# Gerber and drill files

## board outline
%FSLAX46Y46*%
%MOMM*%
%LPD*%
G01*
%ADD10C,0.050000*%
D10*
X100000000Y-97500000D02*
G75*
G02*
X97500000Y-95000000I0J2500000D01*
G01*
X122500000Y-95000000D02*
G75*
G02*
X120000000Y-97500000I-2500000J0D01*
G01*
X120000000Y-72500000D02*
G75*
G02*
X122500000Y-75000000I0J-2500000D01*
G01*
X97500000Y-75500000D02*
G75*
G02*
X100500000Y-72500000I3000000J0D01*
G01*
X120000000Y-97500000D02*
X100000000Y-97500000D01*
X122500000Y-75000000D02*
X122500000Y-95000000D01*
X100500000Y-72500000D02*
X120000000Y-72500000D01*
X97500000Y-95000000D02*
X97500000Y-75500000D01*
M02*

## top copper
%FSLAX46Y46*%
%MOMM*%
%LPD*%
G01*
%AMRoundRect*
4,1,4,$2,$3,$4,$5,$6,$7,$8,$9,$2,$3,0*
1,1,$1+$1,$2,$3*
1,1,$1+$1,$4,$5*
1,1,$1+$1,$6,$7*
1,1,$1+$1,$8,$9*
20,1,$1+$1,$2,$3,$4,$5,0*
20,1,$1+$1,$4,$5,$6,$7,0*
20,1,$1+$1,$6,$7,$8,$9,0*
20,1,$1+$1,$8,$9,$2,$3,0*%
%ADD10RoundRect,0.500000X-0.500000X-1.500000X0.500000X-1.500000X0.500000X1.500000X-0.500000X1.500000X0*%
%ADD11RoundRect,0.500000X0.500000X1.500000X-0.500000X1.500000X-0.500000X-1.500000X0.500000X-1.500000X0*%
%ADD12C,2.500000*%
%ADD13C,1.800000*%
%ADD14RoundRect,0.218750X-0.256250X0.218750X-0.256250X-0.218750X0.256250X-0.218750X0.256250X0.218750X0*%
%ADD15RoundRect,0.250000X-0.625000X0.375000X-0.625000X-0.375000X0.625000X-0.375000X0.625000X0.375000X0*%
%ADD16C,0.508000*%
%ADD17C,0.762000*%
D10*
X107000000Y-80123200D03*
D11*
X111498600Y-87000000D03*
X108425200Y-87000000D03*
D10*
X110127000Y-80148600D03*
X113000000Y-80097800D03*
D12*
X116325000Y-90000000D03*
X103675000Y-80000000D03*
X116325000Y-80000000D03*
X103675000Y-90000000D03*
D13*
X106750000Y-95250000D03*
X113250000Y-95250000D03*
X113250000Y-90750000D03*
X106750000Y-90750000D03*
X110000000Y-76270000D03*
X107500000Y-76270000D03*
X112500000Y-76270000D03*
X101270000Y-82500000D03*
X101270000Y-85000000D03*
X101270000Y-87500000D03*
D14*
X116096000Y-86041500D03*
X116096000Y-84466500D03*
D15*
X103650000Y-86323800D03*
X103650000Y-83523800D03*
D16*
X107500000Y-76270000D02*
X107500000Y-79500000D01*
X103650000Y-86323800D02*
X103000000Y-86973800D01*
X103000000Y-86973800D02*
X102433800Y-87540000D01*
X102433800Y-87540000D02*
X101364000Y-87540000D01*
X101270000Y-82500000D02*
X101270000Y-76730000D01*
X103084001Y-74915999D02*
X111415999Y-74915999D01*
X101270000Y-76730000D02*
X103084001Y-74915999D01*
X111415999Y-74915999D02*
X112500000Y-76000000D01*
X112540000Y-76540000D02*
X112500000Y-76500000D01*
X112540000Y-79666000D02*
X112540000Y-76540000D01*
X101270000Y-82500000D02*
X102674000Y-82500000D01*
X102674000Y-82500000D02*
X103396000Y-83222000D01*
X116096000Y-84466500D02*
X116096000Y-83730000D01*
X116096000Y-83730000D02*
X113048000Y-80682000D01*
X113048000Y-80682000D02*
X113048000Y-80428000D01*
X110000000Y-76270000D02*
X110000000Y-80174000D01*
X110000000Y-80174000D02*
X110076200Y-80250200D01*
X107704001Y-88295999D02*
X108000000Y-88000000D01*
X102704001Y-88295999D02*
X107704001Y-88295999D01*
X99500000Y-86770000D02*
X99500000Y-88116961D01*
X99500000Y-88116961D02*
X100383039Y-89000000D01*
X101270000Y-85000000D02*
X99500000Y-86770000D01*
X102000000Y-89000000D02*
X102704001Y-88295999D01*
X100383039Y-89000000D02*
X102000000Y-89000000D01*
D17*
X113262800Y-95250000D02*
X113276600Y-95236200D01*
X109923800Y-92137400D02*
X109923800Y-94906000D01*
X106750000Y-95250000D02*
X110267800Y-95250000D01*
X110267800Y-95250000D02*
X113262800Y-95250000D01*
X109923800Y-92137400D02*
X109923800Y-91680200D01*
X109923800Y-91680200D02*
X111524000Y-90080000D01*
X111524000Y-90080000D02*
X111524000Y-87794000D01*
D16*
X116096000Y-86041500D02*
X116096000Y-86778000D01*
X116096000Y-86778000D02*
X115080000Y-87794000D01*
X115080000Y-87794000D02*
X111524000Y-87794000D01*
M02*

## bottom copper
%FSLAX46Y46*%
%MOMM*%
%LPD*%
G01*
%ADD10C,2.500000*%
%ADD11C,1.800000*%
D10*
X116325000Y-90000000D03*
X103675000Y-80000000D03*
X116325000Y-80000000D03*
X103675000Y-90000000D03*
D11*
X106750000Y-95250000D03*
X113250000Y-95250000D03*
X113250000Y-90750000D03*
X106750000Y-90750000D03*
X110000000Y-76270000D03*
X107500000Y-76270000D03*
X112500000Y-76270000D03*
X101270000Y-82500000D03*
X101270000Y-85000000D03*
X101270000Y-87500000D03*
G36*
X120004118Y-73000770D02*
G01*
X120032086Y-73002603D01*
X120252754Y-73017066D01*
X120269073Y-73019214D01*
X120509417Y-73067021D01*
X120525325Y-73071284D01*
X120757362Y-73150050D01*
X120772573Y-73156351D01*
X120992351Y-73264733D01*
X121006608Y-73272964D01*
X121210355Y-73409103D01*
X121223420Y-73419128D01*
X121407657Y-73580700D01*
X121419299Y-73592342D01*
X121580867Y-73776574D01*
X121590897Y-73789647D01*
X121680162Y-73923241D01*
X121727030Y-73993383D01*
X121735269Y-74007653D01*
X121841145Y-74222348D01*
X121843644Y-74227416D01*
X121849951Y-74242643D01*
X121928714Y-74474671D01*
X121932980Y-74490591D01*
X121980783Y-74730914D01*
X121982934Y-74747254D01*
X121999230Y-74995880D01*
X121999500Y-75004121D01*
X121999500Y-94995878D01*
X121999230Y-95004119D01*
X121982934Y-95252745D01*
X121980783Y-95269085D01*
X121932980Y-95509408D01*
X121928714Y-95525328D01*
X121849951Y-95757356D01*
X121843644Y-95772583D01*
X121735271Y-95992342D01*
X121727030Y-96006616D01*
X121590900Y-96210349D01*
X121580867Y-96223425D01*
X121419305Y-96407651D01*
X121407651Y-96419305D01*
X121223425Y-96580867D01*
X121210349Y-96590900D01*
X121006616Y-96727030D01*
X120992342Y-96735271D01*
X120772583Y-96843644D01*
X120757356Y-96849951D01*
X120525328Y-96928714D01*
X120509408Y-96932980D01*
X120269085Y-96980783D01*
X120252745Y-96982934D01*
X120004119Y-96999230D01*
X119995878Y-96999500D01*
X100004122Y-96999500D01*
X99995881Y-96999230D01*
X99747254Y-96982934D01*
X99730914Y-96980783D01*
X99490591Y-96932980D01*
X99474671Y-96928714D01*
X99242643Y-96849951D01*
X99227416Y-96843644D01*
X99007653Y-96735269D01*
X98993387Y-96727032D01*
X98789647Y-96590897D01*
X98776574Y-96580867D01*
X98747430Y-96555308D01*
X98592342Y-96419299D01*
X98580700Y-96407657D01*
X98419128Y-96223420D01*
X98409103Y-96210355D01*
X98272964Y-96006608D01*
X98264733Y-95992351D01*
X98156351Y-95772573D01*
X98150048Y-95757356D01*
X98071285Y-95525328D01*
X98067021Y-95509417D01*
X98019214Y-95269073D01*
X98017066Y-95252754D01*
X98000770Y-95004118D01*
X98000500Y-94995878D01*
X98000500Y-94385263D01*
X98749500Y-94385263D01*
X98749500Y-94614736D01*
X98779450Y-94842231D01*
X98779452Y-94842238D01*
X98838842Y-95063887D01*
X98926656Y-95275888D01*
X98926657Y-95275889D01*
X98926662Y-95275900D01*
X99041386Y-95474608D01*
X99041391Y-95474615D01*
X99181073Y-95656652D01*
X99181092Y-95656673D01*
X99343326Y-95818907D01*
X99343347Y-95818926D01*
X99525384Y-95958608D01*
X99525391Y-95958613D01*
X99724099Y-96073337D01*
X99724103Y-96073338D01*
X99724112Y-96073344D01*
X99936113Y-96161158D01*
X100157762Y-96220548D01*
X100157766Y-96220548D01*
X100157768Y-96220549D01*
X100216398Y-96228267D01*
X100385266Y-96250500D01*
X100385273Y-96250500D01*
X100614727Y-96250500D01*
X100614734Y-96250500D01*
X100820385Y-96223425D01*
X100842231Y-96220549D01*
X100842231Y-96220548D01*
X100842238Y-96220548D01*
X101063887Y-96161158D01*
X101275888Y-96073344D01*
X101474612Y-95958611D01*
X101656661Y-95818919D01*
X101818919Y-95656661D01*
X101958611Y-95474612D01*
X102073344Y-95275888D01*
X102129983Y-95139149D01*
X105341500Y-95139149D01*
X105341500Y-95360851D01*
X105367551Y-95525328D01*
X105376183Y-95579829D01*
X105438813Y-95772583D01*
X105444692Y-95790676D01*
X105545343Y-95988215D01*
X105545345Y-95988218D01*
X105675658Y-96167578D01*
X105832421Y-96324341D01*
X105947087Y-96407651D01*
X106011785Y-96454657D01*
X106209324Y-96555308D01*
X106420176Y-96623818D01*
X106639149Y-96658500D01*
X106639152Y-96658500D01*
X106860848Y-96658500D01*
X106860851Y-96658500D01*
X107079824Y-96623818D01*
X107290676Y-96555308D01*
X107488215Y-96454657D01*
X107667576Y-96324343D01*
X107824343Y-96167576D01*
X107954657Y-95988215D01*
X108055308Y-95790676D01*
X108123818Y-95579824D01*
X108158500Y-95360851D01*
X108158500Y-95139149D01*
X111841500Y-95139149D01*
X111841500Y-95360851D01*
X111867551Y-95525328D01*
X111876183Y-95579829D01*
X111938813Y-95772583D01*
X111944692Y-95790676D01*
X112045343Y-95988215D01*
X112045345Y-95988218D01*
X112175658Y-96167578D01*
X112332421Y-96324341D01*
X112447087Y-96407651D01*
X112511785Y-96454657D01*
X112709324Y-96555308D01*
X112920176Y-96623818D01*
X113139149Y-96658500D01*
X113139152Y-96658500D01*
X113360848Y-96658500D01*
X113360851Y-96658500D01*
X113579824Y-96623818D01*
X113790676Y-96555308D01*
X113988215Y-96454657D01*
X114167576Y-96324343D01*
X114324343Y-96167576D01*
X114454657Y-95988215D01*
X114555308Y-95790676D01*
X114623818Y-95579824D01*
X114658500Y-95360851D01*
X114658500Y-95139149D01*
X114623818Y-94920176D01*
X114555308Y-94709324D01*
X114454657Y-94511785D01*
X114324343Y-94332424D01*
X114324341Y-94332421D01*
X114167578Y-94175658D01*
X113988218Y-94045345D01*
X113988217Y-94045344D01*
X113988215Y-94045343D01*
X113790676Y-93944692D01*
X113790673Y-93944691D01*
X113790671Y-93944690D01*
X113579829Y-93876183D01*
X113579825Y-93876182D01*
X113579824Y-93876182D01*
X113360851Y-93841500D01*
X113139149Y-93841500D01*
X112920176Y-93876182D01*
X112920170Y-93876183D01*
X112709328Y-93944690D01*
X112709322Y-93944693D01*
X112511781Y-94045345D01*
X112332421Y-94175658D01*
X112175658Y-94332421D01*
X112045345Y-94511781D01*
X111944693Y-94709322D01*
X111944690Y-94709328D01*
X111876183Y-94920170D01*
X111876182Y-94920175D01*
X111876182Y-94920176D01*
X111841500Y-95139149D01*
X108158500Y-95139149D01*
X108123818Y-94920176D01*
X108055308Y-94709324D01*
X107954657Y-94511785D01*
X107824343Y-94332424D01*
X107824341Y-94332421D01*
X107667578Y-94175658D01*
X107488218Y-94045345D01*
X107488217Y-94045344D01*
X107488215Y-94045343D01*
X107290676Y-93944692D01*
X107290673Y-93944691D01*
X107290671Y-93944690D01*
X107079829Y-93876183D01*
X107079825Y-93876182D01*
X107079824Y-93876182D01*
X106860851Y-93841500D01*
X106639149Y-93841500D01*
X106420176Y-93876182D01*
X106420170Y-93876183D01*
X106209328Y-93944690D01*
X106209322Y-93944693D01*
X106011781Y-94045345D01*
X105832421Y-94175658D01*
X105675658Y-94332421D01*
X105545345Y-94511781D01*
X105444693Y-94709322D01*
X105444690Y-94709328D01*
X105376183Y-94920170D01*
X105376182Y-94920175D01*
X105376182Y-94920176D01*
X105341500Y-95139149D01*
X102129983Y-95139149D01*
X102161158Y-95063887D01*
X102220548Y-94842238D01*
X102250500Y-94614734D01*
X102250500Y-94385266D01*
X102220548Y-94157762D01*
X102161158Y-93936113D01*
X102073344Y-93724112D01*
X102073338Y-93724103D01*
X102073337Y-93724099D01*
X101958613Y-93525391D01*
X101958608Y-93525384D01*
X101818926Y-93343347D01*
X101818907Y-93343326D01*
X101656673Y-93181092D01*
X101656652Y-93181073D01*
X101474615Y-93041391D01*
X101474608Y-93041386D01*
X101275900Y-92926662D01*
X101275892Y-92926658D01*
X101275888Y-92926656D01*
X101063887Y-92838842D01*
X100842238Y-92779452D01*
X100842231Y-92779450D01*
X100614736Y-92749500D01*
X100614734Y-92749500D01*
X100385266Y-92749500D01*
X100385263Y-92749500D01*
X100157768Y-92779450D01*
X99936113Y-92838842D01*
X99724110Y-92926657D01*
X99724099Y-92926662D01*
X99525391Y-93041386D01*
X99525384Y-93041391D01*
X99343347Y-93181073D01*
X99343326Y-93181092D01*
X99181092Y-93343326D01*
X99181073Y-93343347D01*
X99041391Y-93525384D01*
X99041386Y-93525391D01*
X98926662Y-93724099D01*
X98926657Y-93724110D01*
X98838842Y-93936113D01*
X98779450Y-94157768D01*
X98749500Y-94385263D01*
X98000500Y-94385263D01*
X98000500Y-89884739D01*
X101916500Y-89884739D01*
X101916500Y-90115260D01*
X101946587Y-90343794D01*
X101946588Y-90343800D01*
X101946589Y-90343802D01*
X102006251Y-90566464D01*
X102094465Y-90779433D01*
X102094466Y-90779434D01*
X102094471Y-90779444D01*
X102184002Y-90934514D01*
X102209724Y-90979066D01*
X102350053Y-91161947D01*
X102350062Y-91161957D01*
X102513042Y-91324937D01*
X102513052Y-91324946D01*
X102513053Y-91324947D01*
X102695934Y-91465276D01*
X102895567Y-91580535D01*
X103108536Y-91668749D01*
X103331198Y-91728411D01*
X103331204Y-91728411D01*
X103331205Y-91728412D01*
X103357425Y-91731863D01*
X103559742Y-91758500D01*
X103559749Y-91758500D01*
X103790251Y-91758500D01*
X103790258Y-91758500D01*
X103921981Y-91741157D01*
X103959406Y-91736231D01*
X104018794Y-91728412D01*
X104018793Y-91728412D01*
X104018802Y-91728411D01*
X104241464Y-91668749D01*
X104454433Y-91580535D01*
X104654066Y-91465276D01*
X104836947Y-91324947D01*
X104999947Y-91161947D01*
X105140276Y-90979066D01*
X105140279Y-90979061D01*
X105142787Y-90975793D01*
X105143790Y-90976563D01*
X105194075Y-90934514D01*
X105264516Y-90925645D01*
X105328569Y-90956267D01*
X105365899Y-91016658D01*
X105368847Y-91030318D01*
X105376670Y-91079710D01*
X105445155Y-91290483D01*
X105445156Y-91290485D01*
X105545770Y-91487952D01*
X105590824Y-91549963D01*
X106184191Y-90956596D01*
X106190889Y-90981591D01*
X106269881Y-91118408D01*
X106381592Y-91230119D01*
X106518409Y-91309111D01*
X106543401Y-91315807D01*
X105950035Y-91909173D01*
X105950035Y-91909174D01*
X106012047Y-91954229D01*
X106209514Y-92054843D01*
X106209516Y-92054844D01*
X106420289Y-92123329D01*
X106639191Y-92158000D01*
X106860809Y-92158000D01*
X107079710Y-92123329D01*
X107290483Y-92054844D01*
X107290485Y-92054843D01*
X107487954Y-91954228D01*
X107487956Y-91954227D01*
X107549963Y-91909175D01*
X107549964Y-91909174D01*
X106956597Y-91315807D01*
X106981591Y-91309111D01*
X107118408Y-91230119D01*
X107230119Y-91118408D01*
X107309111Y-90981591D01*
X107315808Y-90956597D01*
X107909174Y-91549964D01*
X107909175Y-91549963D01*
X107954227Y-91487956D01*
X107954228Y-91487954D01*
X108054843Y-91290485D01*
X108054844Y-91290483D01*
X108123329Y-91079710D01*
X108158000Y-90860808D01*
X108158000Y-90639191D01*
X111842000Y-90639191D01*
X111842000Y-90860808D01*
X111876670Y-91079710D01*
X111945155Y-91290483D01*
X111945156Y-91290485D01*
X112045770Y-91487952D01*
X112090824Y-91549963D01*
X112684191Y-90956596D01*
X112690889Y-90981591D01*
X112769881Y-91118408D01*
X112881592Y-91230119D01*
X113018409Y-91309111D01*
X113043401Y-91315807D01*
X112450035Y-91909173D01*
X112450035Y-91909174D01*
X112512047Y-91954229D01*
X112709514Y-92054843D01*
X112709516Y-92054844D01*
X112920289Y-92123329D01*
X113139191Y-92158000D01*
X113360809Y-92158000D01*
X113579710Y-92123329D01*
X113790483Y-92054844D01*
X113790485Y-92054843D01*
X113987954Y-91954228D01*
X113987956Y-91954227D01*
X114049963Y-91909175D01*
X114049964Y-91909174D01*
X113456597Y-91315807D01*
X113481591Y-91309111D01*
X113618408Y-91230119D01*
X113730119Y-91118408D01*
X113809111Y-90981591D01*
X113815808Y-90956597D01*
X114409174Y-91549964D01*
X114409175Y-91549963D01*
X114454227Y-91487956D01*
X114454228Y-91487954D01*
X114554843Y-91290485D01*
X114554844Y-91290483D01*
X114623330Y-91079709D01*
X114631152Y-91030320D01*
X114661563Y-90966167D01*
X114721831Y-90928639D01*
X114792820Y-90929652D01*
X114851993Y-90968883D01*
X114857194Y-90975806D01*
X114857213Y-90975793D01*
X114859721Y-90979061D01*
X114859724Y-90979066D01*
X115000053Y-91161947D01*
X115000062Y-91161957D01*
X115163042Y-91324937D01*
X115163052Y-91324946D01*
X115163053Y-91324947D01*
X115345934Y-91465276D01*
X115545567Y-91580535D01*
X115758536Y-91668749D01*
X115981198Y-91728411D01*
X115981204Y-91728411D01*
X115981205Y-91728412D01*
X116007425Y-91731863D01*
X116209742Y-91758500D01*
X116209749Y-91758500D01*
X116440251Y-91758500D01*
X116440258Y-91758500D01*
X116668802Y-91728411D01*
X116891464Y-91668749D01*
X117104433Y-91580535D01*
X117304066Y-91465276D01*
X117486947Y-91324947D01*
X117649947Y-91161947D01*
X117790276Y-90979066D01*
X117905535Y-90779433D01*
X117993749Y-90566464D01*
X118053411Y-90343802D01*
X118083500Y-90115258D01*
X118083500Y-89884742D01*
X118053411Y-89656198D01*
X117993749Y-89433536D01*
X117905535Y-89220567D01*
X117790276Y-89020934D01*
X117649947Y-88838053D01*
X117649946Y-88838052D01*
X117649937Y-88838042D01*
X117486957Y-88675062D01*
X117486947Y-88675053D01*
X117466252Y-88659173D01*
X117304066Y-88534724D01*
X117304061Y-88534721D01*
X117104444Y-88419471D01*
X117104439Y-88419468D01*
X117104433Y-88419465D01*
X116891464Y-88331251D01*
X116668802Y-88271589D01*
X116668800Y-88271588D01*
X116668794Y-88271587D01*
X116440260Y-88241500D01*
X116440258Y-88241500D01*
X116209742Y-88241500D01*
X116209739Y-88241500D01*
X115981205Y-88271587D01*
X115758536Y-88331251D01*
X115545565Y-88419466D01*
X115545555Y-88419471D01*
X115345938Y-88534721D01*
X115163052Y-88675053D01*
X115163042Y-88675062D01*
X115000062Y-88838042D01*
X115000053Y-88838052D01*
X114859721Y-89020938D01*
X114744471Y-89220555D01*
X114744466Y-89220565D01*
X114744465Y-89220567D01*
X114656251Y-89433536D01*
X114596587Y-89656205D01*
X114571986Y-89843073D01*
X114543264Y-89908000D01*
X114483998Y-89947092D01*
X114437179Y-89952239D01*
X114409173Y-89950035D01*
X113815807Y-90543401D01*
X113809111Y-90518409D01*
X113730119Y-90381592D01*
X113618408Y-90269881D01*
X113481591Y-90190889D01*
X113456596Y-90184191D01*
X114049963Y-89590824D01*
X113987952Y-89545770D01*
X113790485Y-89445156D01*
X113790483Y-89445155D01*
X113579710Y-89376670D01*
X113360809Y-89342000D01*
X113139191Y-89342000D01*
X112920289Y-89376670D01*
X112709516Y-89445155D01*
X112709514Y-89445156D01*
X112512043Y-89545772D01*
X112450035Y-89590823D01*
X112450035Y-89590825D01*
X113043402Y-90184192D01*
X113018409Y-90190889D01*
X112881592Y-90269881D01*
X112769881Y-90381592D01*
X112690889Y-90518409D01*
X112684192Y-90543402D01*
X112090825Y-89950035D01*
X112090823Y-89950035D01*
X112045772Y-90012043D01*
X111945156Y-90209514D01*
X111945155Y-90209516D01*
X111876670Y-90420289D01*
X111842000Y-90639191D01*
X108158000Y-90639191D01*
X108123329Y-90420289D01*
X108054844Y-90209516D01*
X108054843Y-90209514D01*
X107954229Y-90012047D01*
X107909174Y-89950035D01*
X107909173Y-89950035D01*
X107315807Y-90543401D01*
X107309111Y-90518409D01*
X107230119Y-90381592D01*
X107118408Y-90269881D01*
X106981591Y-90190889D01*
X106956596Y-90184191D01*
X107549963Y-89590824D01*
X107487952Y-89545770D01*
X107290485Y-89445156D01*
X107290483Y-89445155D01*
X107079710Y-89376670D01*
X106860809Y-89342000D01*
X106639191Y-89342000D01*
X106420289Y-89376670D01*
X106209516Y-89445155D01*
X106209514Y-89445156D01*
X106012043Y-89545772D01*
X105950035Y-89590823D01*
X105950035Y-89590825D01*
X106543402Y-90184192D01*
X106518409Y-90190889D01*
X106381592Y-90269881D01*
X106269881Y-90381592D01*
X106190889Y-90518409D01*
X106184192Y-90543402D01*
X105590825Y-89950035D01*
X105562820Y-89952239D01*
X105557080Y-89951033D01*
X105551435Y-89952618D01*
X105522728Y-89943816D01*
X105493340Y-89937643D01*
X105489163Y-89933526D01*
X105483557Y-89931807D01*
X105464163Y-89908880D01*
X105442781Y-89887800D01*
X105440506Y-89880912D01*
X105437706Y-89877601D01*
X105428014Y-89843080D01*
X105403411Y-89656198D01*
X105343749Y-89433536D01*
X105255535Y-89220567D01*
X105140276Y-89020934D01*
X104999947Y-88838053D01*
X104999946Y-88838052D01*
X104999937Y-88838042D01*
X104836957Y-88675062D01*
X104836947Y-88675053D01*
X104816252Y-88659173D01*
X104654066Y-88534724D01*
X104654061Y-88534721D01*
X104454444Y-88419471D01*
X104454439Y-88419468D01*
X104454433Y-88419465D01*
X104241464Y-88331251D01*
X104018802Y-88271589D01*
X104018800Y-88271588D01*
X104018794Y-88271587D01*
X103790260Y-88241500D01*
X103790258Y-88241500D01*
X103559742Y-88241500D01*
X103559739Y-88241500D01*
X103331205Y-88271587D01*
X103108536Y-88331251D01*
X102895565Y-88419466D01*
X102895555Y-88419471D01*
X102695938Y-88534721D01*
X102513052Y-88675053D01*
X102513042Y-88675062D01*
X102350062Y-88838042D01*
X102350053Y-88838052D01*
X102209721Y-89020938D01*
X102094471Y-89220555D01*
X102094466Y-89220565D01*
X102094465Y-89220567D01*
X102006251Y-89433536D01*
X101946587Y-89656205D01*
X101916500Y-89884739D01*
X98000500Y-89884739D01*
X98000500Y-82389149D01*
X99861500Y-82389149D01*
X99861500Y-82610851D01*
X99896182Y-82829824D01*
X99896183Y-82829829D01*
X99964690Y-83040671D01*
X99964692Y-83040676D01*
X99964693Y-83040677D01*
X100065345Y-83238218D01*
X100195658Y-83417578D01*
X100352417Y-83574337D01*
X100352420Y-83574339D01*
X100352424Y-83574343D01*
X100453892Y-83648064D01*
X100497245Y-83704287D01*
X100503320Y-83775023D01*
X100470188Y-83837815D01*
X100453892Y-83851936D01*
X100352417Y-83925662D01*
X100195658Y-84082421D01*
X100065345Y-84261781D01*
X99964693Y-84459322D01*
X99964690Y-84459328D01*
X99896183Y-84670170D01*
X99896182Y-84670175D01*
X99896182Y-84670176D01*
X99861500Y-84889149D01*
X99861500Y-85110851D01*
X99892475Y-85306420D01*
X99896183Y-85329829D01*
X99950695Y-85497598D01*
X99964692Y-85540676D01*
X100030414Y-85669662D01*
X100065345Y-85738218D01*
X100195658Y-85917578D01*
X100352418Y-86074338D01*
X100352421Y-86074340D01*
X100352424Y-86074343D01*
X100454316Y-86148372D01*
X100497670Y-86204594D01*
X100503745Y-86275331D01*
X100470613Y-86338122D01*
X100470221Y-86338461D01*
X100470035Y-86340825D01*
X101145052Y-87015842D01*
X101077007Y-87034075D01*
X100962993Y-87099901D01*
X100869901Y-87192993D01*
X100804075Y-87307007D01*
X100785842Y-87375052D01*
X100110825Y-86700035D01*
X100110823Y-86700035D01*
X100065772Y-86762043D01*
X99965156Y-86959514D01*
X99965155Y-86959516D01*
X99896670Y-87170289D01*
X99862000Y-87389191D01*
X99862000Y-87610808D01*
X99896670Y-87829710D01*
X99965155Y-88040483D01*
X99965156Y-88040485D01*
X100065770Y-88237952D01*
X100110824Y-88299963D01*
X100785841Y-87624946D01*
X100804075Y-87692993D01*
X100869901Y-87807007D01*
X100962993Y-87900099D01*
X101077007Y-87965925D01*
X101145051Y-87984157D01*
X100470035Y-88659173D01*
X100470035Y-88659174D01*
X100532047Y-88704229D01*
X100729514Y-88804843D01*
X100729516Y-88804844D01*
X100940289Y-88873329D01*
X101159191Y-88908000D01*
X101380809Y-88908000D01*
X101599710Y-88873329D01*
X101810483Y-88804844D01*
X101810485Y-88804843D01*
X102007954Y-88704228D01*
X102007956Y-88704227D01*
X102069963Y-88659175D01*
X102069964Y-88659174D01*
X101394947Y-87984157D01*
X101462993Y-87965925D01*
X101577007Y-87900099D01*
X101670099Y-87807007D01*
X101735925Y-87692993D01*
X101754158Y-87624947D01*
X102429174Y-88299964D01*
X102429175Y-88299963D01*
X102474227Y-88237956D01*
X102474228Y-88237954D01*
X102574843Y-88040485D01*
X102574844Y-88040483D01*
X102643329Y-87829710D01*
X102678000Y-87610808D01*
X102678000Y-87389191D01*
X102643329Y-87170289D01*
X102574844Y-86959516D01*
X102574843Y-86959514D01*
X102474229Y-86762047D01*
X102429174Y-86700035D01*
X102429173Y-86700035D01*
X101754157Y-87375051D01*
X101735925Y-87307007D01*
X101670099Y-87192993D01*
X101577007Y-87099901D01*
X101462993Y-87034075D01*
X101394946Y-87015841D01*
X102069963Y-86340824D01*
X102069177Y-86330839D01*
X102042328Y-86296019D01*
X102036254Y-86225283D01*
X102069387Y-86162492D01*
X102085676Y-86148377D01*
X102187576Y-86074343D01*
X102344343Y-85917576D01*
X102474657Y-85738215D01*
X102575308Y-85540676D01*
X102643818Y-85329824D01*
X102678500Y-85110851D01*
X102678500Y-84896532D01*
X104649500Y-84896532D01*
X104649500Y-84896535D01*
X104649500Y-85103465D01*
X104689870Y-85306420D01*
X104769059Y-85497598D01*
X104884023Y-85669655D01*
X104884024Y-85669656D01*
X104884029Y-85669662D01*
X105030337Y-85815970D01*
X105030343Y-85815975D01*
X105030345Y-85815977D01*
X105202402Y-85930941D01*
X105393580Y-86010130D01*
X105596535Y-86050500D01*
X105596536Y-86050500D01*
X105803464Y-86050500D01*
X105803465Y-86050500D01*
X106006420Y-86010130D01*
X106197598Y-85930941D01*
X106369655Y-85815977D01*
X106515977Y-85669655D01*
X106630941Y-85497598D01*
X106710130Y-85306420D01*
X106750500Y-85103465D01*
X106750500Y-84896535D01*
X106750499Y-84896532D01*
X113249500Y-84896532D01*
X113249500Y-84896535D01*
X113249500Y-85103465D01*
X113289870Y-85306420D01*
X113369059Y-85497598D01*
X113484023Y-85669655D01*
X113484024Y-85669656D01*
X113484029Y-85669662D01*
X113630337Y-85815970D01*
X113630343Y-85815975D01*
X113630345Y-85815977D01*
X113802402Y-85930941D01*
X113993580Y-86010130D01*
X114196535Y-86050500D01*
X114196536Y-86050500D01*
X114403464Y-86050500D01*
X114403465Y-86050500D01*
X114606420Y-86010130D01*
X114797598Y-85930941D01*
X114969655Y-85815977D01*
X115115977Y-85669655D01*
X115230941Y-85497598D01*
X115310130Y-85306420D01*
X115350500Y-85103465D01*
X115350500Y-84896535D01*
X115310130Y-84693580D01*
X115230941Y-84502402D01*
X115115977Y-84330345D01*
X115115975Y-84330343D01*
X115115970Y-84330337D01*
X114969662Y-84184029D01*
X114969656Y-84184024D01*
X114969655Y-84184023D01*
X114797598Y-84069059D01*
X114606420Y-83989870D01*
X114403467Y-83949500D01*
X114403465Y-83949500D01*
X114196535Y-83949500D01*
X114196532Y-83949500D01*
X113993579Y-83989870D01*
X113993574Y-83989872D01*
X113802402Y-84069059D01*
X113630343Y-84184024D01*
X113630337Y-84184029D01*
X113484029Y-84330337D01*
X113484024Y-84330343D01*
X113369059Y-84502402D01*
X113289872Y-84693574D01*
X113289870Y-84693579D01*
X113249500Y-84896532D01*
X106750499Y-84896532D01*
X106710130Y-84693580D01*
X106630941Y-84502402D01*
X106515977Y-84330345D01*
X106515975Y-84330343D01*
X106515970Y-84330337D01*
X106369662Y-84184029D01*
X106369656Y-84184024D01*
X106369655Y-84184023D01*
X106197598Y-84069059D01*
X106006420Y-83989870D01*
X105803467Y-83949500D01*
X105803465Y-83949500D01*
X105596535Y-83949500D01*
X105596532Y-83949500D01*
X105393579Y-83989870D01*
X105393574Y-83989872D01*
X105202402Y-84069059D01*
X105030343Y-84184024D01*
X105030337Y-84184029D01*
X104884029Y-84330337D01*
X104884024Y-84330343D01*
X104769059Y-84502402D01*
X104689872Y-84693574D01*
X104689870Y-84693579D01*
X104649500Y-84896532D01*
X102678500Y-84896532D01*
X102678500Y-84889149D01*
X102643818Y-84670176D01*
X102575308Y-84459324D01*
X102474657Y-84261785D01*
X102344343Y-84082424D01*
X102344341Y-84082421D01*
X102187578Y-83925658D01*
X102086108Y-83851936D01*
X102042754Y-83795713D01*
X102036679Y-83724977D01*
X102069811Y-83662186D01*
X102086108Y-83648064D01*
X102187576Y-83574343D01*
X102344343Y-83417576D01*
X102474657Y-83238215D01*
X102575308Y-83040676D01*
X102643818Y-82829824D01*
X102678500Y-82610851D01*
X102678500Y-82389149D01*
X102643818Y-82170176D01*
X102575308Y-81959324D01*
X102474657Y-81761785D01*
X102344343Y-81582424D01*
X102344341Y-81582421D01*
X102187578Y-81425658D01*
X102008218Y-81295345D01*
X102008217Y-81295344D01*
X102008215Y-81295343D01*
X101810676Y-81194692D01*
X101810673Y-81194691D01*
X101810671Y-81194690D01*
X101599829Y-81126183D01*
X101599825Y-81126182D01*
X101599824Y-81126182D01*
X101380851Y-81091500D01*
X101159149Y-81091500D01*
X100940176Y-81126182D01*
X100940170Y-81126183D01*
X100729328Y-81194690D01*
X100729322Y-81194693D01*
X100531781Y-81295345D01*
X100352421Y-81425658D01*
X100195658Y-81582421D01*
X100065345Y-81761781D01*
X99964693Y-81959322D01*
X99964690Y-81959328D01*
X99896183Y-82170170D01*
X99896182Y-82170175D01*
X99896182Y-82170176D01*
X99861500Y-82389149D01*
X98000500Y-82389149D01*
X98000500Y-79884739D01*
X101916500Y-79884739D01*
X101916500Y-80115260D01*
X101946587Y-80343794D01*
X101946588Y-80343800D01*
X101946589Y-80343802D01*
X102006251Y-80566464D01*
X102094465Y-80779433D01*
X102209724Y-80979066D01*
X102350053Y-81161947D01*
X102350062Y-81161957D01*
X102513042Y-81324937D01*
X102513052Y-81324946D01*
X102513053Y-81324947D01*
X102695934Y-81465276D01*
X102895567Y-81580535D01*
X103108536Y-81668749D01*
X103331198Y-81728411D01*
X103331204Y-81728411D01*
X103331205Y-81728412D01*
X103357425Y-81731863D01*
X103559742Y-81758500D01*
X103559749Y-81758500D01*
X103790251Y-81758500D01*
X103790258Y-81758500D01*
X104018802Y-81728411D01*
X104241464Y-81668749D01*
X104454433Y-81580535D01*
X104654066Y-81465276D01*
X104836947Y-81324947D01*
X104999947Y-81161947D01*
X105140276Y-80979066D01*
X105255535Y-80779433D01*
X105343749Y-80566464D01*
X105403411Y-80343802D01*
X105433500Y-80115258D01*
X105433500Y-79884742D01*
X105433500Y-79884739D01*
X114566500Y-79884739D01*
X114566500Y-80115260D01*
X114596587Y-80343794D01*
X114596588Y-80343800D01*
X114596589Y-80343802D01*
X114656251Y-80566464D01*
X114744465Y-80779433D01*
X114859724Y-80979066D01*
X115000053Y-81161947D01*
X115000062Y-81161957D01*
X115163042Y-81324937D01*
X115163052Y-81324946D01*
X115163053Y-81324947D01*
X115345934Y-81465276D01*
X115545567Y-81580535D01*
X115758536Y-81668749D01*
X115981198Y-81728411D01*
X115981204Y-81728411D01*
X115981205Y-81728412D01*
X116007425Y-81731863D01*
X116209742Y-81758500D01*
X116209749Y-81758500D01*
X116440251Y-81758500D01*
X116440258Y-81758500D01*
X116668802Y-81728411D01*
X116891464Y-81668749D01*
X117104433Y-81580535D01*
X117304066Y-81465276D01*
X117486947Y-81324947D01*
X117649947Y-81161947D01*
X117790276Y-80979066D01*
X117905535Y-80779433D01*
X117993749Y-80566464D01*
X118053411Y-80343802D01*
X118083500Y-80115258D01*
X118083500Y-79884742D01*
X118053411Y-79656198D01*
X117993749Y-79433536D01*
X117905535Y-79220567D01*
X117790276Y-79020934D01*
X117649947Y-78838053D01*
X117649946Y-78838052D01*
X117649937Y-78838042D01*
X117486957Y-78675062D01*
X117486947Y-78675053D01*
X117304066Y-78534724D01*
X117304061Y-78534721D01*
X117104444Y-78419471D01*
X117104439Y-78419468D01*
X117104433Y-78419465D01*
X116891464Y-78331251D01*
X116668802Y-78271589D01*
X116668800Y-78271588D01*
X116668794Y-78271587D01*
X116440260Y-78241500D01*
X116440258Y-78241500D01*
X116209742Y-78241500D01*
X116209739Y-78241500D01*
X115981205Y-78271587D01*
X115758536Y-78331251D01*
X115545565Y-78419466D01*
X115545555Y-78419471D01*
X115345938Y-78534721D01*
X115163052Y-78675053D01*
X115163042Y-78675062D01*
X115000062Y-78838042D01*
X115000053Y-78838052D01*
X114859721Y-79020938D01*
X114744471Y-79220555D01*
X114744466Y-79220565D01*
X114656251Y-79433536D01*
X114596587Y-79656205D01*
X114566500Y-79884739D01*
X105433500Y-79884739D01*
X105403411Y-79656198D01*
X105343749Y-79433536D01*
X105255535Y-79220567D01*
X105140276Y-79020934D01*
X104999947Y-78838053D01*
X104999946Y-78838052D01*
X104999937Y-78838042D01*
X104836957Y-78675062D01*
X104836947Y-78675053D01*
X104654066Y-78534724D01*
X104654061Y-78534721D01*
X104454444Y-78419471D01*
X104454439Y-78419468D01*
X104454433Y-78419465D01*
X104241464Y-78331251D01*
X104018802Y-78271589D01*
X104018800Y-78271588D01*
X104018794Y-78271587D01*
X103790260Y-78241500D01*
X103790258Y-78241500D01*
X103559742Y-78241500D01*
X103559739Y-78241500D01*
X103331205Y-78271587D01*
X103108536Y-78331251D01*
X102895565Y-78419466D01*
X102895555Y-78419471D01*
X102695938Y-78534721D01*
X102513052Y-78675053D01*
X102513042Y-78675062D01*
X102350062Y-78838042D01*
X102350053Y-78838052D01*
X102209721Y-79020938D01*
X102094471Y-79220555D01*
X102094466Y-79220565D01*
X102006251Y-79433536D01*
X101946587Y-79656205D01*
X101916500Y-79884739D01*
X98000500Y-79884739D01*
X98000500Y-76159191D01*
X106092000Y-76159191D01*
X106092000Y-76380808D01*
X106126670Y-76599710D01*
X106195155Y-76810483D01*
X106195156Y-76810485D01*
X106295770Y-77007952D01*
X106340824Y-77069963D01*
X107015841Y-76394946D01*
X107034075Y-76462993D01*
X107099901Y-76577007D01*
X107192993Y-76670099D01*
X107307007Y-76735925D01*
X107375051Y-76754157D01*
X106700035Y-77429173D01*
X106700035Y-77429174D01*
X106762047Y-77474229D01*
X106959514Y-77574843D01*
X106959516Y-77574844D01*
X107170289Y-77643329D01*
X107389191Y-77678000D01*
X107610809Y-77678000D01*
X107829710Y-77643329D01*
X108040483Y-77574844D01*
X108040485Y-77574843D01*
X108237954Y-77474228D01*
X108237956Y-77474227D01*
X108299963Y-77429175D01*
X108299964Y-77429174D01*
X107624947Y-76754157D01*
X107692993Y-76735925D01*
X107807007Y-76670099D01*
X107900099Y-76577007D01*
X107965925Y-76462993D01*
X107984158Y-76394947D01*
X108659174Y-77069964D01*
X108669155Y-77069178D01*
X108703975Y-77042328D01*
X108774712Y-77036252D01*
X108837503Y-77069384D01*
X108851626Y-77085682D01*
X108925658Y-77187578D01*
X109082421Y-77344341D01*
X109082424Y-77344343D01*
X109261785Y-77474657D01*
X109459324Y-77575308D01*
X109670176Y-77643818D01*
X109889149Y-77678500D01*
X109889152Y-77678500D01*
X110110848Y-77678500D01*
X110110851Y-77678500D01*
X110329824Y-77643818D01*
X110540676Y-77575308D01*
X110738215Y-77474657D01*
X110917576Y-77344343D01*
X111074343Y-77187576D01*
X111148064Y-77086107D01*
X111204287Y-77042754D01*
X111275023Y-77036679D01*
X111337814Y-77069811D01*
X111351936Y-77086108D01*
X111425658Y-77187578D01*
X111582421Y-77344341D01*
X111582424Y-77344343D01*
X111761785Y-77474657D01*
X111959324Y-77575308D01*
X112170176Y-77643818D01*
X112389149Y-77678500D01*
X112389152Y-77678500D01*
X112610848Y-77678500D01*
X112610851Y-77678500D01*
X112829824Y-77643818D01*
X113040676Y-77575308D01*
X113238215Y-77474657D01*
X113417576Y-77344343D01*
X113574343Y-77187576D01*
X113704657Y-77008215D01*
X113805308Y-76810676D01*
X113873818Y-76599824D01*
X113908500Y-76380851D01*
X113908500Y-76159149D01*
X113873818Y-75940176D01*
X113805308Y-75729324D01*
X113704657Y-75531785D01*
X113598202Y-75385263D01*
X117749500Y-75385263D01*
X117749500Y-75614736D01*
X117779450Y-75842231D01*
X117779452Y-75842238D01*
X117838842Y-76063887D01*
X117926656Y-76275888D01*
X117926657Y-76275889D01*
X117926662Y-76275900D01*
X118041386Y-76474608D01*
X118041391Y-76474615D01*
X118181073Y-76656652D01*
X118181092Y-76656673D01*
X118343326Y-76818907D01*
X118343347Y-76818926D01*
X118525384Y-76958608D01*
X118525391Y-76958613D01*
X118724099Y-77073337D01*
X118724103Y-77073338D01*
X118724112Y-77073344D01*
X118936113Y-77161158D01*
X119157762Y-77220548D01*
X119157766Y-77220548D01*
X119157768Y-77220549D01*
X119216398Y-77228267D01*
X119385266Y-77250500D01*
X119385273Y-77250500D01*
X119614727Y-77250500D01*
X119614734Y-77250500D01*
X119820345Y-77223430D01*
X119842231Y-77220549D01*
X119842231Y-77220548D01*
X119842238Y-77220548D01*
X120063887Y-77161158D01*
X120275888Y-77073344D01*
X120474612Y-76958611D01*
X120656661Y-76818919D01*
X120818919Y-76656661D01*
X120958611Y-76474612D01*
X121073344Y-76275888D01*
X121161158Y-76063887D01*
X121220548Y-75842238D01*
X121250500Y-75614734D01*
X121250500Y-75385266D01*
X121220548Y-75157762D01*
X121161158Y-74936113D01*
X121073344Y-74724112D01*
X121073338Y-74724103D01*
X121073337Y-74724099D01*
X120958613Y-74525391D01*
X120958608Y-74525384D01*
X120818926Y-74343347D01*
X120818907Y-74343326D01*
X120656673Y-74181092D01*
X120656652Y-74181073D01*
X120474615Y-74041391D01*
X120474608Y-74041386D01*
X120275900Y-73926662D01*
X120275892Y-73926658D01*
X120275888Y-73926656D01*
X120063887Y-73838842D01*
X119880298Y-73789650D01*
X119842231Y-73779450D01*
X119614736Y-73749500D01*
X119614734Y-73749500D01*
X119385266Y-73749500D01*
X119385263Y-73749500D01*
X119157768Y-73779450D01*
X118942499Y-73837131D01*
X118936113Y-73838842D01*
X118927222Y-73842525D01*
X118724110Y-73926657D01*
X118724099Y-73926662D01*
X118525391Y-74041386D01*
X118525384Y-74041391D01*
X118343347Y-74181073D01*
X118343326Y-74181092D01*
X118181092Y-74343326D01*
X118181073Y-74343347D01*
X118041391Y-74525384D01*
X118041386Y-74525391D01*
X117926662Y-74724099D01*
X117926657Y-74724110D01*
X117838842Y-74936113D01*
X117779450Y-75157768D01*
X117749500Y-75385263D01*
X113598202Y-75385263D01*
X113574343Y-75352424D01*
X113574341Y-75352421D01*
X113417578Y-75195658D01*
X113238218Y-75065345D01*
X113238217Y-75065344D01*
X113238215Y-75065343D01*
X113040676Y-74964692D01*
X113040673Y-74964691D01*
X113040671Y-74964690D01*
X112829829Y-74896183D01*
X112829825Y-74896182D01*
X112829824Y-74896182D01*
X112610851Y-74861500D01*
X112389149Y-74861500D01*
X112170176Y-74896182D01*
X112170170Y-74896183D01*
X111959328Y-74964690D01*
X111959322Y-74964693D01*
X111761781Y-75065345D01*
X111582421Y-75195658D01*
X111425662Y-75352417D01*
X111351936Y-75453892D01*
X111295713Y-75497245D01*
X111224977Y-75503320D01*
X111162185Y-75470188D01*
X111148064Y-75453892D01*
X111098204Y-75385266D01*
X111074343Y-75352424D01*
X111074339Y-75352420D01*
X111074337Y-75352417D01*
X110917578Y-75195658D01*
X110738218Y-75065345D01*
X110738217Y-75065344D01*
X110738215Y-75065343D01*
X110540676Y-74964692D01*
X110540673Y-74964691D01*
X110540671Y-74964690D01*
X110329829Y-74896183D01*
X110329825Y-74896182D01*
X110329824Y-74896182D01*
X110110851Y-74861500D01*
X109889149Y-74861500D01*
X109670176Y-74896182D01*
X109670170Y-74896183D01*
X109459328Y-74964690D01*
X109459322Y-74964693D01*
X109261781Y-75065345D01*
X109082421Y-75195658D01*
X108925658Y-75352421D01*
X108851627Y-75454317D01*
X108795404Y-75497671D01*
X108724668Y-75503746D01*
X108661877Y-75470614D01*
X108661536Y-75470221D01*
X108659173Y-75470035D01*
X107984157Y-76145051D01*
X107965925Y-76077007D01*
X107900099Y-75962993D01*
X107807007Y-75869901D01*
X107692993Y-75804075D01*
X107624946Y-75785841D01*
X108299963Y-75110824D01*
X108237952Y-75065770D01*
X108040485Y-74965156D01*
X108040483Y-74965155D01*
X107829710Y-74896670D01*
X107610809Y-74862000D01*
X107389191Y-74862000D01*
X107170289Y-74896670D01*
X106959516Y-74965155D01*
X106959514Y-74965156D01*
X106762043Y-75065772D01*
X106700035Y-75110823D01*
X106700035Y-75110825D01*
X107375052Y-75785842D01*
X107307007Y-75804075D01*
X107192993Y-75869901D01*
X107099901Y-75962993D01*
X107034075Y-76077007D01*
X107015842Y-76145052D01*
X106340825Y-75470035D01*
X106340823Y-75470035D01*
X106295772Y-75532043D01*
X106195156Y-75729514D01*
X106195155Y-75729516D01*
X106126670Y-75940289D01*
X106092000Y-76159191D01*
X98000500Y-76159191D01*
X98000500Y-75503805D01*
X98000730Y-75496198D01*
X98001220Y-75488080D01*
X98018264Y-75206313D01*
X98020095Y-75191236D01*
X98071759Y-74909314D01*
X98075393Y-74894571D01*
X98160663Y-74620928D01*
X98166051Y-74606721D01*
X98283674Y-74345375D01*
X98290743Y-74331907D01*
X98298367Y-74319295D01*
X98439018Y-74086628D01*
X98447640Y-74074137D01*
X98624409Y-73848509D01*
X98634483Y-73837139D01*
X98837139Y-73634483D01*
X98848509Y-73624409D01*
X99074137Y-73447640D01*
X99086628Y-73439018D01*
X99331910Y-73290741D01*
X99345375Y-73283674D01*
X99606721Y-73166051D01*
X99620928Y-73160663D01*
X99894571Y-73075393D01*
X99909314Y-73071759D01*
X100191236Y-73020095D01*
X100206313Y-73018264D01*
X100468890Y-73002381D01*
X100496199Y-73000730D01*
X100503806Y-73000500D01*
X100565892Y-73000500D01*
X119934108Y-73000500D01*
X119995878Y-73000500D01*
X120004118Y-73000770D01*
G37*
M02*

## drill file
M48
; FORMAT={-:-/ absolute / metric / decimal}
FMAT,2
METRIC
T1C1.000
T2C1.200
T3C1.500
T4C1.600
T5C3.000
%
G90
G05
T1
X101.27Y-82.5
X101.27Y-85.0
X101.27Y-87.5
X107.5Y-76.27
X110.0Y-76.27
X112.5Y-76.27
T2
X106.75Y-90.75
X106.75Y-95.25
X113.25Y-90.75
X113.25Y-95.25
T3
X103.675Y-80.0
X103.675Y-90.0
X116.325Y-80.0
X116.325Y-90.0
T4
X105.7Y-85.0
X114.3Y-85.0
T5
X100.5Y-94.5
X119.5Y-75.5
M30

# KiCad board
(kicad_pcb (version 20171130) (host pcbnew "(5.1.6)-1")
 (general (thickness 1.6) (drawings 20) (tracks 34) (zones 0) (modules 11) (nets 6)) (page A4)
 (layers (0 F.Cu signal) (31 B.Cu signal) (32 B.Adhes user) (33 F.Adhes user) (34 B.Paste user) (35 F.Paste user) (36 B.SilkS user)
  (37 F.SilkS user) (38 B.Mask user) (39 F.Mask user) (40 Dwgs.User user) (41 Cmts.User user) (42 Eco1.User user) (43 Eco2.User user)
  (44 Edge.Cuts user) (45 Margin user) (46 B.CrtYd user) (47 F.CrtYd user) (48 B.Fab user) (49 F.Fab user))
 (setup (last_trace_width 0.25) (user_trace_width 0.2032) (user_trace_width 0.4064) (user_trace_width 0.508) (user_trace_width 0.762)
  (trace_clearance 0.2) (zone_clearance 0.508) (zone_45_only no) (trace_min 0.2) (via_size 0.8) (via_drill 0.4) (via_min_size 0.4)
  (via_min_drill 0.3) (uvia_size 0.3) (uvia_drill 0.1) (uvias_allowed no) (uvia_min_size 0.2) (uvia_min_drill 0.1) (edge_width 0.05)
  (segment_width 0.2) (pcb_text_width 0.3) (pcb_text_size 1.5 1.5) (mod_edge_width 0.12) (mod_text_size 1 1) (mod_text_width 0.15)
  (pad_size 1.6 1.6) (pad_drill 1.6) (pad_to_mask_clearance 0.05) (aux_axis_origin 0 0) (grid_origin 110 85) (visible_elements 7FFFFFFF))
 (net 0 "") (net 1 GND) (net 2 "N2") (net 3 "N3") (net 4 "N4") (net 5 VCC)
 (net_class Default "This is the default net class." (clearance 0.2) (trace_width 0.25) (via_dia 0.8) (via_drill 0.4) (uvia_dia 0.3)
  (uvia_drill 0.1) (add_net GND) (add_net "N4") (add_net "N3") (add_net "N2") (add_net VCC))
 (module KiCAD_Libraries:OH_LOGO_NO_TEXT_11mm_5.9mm (layer B.Cu) (at 110 81.952)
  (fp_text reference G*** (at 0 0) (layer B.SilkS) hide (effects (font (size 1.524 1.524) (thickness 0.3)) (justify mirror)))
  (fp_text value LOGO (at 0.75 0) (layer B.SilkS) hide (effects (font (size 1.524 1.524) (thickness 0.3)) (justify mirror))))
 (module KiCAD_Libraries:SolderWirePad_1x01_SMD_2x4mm (layer F.Cu) (at 107 80.1232)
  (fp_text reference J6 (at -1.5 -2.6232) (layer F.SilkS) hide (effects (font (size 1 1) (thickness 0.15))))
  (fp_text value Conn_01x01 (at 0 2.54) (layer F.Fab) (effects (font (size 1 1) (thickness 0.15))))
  (pad 1 smd roundrect (at 0 0) (size 2 4) (layers F.Cu F.Paste F.Mask) (roundrect_rratio 0.25) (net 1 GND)))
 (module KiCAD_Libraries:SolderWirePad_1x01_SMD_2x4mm (layer F.Cu) (at 111.4986 87 180)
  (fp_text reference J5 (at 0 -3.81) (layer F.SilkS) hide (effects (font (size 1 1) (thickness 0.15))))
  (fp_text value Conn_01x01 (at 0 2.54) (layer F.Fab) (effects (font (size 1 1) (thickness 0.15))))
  (pad 1 smd roundrect (at 0 0 180) (size 2 4) (layers F.Cu F.Paste F.Mask) (roundrect_rratio 0.25) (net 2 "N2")))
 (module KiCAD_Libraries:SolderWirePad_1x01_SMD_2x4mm (layer F.Cu) (at 108.4252 87 180)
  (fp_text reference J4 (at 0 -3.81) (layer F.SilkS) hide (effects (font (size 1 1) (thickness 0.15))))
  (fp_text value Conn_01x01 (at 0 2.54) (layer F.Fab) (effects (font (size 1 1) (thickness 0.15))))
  (pad 1 smd roundrect (at 0 0 180) (size 2 4) (layers F.Cu F.Paste F.Mask) (roundrect_rratio 0.25) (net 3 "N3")))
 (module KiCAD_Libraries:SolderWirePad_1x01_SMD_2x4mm (layer F.Cu) (at 110.127 80.1486)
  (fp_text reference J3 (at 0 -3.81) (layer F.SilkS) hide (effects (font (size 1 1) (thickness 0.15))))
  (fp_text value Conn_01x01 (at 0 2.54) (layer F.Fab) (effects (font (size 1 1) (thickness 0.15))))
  (pad 1 smd roundrect (at 0 0) (size 2 4) (layers F.Cu F.Paste F.Mask) (roundrect_rratio 0.25) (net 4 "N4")))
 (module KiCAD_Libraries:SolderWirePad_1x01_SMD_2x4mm (layer F.Cu) (at 113 80.0978)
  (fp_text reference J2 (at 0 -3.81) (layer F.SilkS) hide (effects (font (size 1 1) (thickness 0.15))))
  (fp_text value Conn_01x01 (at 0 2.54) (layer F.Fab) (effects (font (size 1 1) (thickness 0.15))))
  (pad 1 smd roundrect (at 0 0) (size 2 4) (layers F.Cu F.Paste F.Mask) (roundrect_rratio 0.25) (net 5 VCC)))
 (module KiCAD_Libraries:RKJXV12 (layer B.Cu) (at 110 85 180)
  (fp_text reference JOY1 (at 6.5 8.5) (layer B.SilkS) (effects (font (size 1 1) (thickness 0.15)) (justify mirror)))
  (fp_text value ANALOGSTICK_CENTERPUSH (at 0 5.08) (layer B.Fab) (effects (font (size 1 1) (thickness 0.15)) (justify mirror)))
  (pad "" np_thru_hole circle (at 4.3 0 180) (size 1.6 1.6) (drill 1.6) (layers *.Cu *.Mask))
  (pad "" np_thru_hole circle (at -4.3 0) (size 1.6 1.6) (drill 1.6) (layers *.Cu *.Mask))
  (pad MNT1 thru_hole circle (at -6.325 -5 180) (size 2.5 2.5) (drill 1.5) (layers *.Cu *.Mask))
  (pad MNT1 thru_hole circle (at 6.325 5) (size 2.5 2.5) (drill 1.5) (layers *.Cu *.Mask))
  (pad MNT1 thru_hole circle (at -6.325 5) (size 2.5 2.5) (drill 1.5) (layers *.Cu *.Mask))
  (pad MNT1 thru_hole circle (at 6.325 -5 180) (size 2.5 2.5) (drill 1.5) (layers *.Cu *.Mask))
  (pad d thru_hole circle (at 3.25 -10.25 180) (size 1.8 1.8) (drill 1.2) (layers *.Cu *.Mask) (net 2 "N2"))
  (pad b thru_hole circle (at -3.25 -10.25 180) (size 1.8 1.8) (drill 1.2) (layers *.Cu *.Mask) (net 2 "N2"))
  (pad a thru_hole circle (at -3.25 -5.75 180) (size 1.8 1.8) (drill 1.2) (layers *.Cu *.Mask) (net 1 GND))
  (pad c thru_hole circle (at 3.25 -5.75 180) (size 1.8 1.8) (drill 1.2) (layers *.Cu *.Mask) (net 1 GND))
  (pad 5 thru_hole circle (at 0 8.73 90) (size 1.8 1.8) (drill 1) (layers *.Cu *.Mask) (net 4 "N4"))
  (pad 4 thru_hole circle (at 2.5 8.73 90) (size 1.8 1.8) (drill 1) (layers *.Cu *.Mask) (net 1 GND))
  (pad 6 thru_hole circle (at -2.5 8.73 90) (size 1.8 1.8) (drill 1) (layers *.Cu *.Mask) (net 5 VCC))
  (pad 3 thru_hole circle (at 8.73 2.5 180) (size 1.8 1.8) (drill 1) (layers *.Cu *.Mask) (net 5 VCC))
  (pad 2 thru_hole circle (at 8.73 0 180) (size 1.8 1.8) (drill 1) (layers *.Cu *.Mask) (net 3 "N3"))
  (pad 1 thru_hole circle (at 8.73 -2.5 180) (size 1.8 1.8) (drill 1) (layers *.Cu *.Mask) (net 1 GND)))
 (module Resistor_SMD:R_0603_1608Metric (layer F.Cu) (at 116.096 85.254 270)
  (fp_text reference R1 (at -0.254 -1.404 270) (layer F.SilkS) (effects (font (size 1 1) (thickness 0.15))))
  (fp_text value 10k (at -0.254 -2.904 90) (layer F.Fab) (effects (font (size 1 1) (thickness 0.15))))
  (pad 2 smd roundrect (at 0.7875 0 270) (size 0.875 0.95) (layers F.Cu F.Paste F.Mask) (roundrect_rratio 0.25) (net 2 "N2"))
  (pad 1 smd roundrect (at -0.7875 0 270) (size 0.875 0.95) (layers F.Cu F.Paste F.Mask) (roundrect_rratio 0.25) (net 5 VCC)))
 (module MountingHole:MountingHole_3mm (layer F.Cu) (at 119.5 75.5)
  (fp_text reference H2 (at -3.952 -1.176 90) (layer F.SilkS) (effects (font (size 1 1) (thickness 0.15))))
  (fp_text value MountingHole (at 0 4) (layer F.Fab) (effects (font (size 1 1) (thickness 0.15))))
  (pad 1 np_thru_hole circle (at 0 0) (size 3 3) (drill 3) (layers *.Cu *.Mask)))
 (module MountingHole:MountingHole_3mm (layer F.Cu) (at 100.5 94.5)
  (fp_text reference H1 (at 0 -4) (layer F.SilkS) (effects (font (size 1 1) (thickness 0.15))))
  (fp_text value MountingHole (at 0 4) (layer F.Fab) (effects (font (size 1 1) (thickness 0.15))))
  (pad 1 np_thru_hole circle (at 0 0) (size 3 3) (drill 3) (layers *.Cu *.Mask)))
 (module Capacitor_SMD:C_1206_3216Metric (layer F.Cu) (at 103.65 84.9238 270)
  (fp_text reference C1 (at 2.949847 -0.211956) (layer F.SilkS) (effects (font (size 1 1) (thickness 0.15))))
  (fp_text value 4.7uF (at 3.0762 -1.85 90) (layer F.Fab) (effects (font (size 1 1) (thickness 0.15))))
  (pad 2 smd roundrect (at 1.4 0 270) (size 1.25 1.75) (layers F.Cu F.Paste F.Mask) (roundrect_rratio 0.2) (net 1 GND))
  (pad 1 smd roundrect (at -1.4 0 270) (size 1.25 1.75) (layers F.Cu F.Paste F.Mask) (roundrect_rratio 0.2) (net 5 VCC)))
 (gr_arc (start 100 95) (end 97.5 95) (angle -90) (layer Edge.Cuts) (width 0.05))
 (gr_arc (start 120 95) (end 120 97.5) (angle -90) (layer Edge.Cuts) (width 0.05))
 (gr_arc (start 120 75) (end 122.5 75) (angle -90) (layer Edge.Cuts) (width 0.05))
 (gr_arc (start 100.5 75.5) (end 100.5 72.5) (angle -90) (layer Edge.Cuts) (width 0.05))
 (gr_line (start 120 97.5) (end 100 97.5) (layer Edge.Cuts) (width 0.05))
 (gr_line (start 122.5 75) (end 122.5 95) (layer Edge.Cuts) (width 0.05))
 (gr_line (start 100.5 72.5) (end 120 72.5) (layer Edge.Cuts) (width 0.05))
 (gr_line (start 97.5 95) (end 97.5 75.5) (layer Edge.Cuts) (width 0.05))
 (segment (start 107.5 76.27) (end 107.5 79.5) (width 0.508) (layer F.Cu) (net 1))
 (segment (start 103.65 86.3238) (end 103 86.9738) (width 0.508) (layer F.Cu) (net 1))
 (segment (start 103 86.9738) (end 102.4338 87.54) (width 0.508) (layer F.Cu) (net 1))
 (segment (start 102.4338 87.54) (end 101.364 87.54) (width 0.508) (layer F.Cu) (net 1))
 (segment (start 101.27 82.5) (end 101.27 76.73) (width 0.508) (layer F.Cu) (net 5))
 (segment (start 103.084001 74.915999) (end 111.415999 74.915999) (width 0.508) (layer F.Cu) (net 5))
 (segment (start 101.27 76.73) (end 103.084001 74.915999) (width 0.508) (layer F.Cu) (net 5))
 (segment (start 111.415999 74.915999) (end 112.5 76) (width 0.508) (layer F.Cu) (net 5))
 (segment (start 112.54 76.54) (end 112.5 76.5) (width 0.508) (layer F.Cu) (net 5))
 (segment (start 112.54 79.666) (end 112.54 76.54) (width 0.508) (layer F.Cu) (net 5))
 (segment (start 101.27 82.5) (end 102.674 82.5) (width 0.508) (layer F.Cu) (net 5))
 (segment (start 102.674 82.5) (end 103.396 83.222) (width 0.508) (layer F.Cu) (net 5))
 (segment (start 116.096 84.4665) (end 116.096 83.73) (width 0.508) (layer F.Cu) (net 5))
 (segment (start 116.096 83.73) (end 113.048 80.682) (width 0.508) (layer F.Cu) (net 5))
 (segment (start 113.048 80.682) (end 113.048 80.428) (width 0.508) (layer F.Cu) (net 5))
 (segment (start 110 76.27) (end 110 80.174) (width 0.508) (layer F.Cu) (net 4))
 (segment (start 110 80.174) (end 110.0762 80.2502) (width 0.508) (layer F.Cu) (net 4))
 (segment (start 107.704001 88.295999) (end 108 88) (width 0.508) (layer F.Cu) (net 3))
 (segment (start 102.704001 88.295999) (end 107.704001 88.295999) (width 0.508) (layer F.Cu) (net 3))
 (segment (start 99.5 86.77) (end 99.5 88.116961) (width 0.508) (layer F.Cu) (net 3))
 (segment (start 99.5 88.116961) (end 100.383039 89) (width 0.508) (layer F.Cu) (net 3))
 (segment (start 101.27 85) (end 99.5 86.77) (width 0.508) (layer F.Cu) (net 3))
 (segment (start 102 89) (end 102.704001 88.295999) (width 0.508) (layer F.Cu) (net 3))
 (segment (start 100.383039 89) (end 102 89) (width 0.508) (layer F.Cu) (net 3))
 (segment (start 113.2628 95.25) (end 113.2766 95.2362) (width 0.762) (layer F.Cu) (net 2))
 (segment (start 109.9238 92.1374) (end 109.9238 94.906) (width 0.762) (layer F.Cu) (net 2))
 (segment (start 106.75 95.25) (end 110.2678 95.25) (width 0.762) (layer F.Cu) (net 2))
 (segment (start 110.2678 95.25) (end 113.2628 95.25) (width 0.762) (layer F.Cu) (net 2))
 (segment (start 109.9238 92.1374) (end 109.9238 91.6802) (width 0.762) (layer F.Cu) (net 2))
 (segment (start 109.9238 91.6802) (end 111.524 90.08) (width 0.762) (layer F.Cu) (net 2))
 (segment (start 111.524 90.08) (end 111.524 87.794) (width 0.762) (layer F.Cu) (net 2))
 (segment (start 116.096 86.0415) (end 116.096 86.778) (width 0.508) (layer F.Cu) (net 2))
 (segment (start 116.096 86.778) (end 115.08 87.794) (width 0.508) (layer F.Cu) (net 2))
 (segment (start 115.08 87.794) (end 111.524 87.794) (width 0.508) (layer F.Cu) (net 2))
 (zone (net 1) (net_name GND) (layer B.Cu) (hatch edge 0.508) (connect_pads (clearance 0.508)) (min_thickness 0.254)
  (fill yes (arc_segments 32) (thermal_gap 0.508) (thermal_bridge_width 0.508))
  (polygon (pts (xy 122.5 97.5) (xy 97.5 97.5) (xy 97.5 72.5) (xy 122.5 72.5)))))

